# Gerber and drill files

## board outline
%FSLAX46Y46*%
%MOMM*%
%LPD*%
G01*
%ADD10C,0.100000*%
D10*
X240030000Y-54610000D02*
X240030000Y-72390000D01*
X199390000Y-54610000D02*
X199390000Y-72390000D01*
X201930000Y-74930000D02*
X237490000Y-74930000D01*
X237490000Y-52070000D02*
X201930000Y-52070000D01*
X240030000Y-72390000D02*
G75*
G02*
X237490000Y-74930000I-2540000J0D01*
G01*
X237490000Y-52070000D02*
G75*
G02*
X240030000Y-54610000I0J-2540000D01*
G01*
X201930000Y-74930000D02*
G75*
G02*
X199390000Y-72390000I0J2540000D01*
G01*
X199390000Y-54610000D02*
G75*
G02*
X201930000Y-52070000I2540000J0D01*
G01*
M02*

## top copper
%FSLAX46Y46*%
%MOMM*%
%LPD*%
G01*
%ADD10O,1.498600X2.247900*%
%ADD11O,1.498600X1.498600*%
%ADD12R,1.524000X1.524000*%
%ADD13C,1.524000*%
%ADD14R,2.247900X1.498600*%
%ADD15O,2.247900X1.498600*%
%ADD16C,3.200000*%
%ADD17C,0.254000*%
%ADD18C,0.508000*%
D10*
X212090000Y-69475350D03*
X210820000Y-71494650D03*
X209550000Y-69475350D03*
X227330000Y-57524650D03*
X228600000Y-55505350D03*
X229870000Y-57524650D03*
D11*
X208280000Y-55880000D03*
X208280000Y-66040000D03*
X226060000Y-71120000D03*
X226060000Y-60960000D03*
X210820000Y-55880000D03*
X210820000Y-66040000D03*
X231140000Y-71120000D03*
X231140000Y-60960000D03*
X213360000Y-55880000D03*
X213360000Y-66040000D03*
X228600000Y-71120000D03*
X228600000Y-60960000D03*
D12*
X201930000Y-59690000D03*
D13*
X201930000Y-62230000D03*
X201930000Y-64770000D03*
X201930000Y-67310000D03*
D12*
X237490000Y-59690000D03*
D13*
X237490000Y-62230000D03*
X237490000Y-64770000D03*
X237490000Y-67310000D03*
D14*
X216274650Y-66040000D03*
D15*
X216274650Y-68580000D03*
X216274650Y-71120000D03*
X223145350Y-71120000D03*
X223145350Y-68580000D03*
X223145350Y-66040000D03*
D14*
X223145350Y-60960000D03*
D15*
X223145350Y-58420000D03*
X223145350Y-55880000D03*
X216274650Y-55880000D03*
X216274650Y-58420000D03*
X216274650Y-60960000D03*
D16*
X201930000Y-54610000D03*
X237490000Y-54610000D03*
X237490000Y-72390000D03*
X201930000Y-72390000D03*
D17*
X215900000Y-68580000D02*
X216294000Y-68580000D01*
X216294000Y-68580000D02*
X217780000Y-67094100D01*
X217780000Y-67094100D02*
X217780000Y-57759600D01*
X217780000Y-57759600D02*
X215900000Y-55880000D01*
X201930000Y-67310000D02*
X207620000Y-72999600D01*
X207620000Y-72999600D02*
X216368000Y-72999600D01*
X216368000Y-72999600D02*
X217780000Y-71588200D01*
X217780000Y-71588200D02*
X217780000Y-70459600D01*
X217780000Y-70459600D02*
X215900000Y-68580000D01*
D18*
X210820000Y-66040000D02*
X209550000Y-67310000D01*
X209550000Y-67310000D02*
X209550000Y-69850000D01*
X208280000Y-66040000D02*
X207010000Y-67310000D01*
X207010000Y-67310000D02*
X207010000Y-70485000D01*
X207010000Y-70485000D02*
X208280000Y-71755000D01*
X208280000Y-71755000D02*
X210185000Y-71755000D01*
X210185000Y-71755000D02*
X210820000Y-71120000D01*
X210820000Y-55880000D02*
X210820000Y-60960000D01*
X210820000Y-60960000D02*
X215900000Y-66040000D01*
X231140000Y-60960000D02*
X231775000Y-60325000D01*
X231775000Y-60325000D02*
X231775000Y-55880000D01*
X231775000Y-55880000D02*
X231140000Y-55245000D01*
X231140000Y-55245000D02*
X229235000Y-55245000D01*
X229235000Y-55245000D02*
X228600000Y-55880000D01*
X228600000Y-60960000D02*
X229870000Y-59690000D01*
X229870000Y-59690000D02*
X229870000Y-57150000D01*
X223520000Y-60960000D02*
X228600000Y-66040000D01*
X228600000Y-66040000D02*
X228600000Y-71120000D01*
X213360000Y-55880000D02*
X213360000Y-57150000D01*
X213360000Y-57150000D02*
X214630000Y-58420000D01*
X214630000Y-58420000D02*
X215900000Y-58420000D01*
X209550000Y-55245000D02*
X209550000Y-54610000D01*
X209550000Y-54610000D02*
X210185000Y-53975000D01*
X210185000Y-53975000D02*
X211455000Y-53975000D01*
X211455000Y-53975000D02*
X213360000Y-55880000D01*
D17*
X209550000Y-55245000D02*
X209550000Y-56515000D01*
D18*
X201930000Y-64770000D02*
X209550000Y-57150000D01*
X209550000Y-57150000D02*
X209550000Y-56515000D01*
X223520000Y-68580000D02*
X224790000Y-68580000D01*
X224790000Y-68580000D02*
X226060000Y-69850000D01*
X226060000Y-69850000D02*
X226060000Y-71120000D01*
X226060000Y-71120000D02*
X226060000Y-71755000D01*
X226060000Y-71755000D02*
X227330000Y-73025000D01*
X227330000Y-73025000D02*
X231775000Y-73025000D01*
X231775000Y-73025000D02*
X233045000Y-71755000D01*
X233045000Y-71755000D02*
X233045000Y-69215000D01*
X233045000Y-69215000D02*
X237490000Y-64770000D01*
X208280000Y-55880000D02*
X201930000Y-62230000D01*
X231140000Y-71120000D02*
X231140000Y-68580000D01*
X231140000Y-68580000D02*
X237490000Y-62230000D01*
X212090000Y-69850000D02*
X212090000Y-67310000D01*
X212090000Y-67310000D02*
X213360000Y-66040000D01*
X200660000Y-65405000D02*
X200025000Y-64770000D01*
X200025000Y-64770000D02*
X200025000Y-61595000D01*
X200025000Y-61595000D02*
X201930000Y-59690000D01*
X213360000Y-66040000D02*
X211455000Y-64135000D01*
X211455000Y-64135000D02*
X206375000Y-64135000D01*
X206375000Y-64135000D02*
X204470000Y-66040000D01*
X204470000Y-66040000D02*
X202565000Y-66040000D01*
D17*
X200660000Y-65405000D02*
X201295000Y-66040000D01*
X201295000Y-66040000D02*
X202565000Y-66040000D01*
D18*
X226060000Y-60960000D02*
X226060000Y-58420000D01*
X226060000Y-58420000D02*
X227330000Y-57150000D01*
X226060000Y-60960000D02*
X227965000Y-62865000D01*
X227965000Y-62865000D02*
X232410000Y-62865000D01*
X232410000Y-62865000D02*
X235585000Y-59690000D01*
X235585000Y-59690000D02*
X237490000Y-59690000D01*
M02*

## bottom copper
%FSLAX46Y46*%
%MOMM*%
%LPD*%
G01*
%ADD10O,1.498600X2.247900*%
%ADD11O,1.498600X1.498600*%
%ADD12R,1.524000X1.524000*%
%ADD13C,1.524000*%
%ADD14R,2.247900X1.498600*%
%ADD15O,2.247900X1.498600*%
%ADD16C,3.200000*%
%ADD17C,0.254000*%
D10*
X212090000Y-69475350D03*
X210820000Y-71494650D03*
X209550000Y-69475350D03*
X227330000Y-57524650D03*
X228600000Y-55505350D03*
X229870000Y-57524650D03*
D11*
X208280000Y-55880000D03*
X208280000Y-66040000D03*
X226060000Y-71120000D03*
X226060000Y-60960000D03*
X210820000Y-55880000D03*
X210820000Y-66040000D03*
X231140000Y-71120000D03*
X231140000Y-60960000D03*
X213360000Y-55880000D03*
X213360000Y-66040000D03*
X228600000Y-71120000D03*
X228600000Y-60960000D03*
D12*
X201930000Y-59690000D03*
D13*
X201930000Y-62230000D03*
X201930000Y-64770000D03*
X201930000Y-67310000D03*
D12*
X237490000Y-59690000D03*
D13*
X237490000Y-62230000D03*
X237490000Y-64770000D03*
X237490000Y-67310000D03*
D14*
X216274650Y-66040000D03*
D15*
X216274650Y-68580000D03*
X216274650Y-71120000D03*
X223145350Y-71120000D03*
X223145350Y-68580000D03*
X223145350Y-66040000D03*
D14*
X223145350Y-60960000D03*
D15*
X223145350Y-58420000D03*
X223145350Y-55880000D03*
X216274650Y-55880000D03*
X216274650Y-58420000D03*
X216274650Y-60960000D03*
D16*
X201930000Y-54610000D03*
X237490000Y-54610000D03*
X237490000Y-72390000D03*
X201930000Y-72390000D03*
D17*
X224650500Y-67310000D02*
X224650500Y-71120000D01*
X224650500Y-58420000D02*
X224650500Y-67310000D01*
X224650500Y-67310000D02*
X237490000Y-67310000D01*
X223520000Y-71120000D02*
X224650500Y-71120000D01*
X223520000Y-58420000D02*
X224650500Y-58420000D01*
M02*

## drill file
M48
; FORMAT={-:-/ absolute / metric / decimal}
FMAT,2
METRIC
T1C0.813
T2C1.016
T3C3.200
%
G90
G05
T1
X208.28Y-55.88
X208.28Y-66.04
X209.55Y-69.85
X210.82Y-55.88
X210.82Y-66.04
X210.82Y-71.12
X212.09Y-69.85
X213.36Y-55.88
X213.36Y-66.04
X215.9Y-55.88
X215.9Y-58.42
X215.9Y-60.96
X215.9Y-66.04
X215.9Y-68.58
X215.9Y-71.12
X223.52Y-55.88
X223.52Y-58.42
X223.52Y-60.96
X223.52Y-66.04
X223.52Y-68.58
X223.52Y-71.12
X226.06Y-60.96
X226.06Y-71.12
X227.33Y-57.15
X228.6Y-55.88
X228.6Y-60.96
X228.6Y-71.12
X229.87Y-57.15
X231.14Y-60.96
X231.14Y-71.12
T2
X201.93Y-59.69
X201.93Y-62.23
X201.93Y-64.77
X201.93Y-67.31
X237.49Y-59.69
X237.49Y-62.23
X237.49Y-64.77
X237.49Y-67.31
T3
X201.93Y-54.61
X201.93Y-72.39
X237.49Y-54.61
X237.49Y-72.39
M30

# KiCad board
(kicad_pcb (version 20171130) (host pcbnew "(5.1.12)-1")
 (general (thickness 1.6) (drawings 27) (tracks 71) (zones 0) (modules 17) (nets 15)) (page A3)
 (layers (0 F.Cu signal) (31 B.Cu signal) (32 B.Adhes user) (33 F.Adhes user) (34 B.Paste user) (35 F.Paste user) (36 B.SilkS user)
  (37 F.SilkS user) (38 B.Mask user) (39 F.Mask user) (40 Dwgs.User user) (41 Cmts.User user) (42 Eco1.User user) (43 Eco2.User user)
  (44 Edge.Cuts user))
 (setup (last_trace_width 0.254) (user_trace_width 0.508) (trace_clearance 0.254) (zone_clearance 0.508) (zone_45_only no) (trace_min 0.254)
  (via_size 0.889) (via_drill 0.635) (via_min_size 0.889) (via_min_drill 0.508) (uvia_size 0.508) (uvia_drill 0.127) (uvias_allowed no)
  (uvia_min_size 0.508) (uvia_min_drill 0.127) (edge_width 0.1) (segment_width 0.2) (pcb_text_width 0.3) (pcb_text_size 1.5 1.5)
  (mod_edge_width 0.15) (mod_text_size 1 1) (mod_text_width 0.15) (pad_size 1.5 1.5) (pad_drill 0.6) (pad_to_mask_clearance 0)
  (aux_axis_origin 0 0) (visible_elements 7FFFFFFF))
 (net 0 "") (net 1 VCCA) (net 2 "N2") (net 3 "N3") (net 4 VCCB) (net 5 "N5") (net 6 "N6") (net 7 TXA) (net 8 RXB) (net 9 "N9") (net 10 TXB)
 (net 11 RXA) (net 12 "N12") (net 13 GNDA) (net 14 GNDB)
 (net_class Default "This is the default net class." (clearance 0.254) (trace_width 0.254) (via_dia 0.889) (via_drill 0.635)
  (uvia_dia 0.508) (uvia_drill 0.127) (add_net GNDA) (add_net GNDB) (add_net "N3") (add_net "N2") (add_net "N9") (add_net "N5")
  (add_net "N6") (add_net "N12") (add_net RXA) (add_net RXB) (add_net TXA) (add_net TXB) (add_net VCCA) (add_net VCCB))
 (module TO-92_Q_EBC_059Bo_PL (layer F.Cu) (at 212.09 69.85)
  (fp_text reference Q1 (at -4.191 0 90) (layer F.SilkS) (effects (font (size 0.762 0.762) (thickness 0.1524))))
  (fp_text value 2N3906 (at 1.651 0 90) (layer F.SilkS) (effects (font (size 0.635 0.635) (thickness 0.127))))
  (pad 1 thru_hole oval (at 0 0) (size 1.4986 2.2479) (drill 0.8128 (offset 0 -0.37465)) (layers *.Cu *.Mask F.SilkS) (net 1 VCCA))
  (pad 2 thru_hole oval (at -1.27 1.27) (size 1.4986 2.2479) (drill 0.8128 (offset 0 0.37465)) (layers *.Cu *.Mask F.SilkS) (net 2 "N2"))
  (pad 3 thru_hole oval (at -2.54 0) (size 1.4986 2.2479) (drill 0.8128 (offset 0 -0.37465)) (layers *.Cu *.Mask F.SilkS) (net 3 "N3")))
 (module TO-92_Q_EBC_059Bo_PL (layer F.Cu) (at 227.33 57.15 180)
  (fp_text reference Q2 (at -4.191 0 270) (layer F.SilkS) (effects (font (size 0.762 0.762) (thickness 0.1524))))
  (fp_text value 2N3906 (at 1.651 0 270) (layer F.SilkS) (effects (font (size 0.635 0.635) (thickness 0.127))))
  (pad 1 thru_hole oval (at 0 0 180) (size 1.4986 2.2479) (drill 0.8128 (offset 0 -0.37465)) (layers *.Cu *.Mask F.SilkS) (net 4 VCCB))
  (pad 2 thru_hole oval (at -1.27 1.27 180) (size 1.4986 2.2479) (drill 0.8128 (offset 0 0.37465)) (layers *.Cu *.Mask F.SilkS) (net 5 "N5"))
  (pad 3 thru_hole oval (at -2.54 0 180) (size 1.4986 2.2479) (drill 0.8128 (offset 0 -0.37465)) (layers *.Cu *.Mask F.SilkS) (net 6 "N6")))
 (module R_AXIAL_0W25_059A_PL (layer F.Cu) (at 208.28 55.88 270) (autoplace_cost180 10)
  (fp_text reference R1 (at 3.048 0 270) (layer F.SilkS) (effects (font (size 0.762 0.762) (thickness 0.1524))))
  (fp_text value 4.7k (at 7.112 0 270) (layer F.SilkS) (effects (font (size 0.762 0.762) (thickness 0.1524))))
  (pad 1 thru_hole oval (at 0 0 270) (size 1.4986 1.4986) (drill 0.8128) (layers *.Cu *.Mask F.SilkS) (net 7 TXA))
  (pad 2 thru_hole oval (at 10.16 0 270) (size 1.4986 1.4986) (drill 0.8128) (layers *.Cu *.Mask F.SilkS) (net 2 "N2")))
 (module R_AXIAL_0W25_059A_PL (layer F.Cu) (at 226.06 71.12 90) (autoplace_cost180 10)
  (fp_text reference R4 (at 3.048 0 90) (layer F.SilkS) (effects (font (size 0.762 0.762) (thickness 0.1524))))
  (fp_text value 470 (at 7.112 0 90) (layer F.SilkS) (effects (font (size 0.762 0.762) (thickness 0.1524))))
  (pad 1 thru_hole oval (at 0 0 90) (size 1.4986 1.4986) (drill 0.8128) (layers *.Cu *.Mask F.SilkS) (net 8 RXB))
  (pad 2 thru_hole oval (at 10.16 0 90) (size 1.4986 1.4986) (drill 0.8128) (layers *.Cu *.Mask F.SilkS) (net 4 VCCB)))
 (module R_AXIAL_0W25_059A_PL (layer F.Cu) (at 210.82 55.88 270) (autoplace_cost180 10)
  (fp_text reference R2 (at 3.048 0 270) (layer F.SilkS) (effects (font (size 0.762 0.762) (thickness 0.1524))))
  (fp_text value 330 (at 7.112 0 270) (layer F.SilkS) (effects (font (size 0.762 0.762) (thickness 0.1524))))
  (pad 1 thru_hole oval (at 0 0 270) (size 1.4986 1.4986) (drill 0.8128) (layers *.Cu *.Mask F.SilkS) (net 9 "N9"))
  (pad 2 thru_hole oval (at 10.16 0 270) (size 1.4986 1.4986) (drill 0.8128) (layers *.Cu *.Mask F.SilkS) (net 3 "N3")))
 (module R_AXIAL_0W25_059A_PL (layer F.Cu) (at 231.14 71.12 90) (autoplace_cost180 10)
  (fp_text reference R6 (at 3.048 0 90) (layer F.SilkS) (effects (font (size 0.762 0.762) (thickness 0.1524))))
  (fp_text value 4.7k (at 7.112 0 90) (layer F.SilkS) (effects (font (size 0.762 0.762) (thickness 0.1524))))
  (pad 1 thru_hole oval (at 0 0 90) (size 1.4986 1.4986) (drill 0.8128) (layers *.Cu *.Mask F.SilkS) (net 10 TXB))
  (pad 2 thru_hole oval (at 10.16 0 90) (size 1.4986 1.4986) (drill 0.8128) (layers *.Cu *.Mask F.SilkS) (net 5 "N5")))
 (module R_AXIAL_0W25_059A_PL (layer F.Cu) (at 213.36 55.88 270) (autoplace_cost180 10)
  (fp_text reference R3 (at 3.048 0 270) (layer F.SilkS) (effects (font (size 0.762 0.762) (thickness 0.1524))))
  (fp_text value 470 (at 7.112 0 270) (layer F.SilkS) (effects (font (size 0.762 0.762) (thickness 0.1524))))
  (pad 1 thru_hole oval (at 0 0 270) (size 1.4986 1.4986) (drill 0.8128) (layers *.Cu *.Mask F.SilkS) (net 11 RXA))
  (pad 2 thru_hole oval (at 10.16 0 270) (size 1.4986 1.4986) (drill 0.8128) (layers *.Cu *.Mask F.SilkS) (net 1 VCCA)))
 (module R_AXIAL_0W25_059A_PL (layer F.Cu) (at 228.6 71.12 90) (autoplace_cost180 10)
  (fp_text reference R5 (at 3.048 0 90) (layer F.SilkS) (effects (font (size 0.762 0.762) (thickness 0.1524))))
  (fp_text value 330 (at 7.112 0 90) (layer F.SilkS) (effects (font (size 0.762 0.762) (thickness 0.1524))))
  (pad 1 thru_hole oval (at 0 0 90) (size 1.4986 1.4986) (drill 0.8128) (layers *.Cu *.Mask F.SilkS) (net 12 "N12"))
  (pad 2 thru_hole oval (at 10.16 0 90) (size 1.4986 1.4986) (drill 0.8128) (layers *.Cu *.Mask F.SilkS) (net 6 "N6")))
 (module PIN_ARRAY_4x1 (layer F.Cu) (at 201.93 63.5 270)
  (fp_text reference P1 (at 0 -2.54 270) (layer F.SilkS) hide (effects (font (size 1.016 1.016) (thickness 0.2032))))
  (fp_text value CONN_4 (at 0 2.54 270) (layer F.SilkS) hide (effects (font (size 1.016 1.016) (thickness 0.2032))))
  (pad 1 thru_hole rect (at -3.81 0 270) (size 1.524 1.524) (drill 1.016) (layers *.Cu *.Mask F.SilkS) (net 1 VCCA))
  (pad 2 thru_hole circle (at -1.27 0 270) (size 1.524 1.524) (drill 1.016) (layers *.Cu *.Mask F.SilkS) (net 7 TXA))
  (pad 3 thru_hole circle (at 1.27 0 270) (size 1.524 1.524) (drill 1.016) (layers *.Cu *.Mask F.SilkS) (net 11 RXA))
  (pad 4 thru_hole circle (at 3.81 0 270) (size 1.524 1.524) (drill 1.016) (layers *.Cu *.Mask F.SilkS) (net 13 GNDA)))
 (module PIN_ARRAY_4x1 (layer F.Cu) (at 237.49 63.5 270)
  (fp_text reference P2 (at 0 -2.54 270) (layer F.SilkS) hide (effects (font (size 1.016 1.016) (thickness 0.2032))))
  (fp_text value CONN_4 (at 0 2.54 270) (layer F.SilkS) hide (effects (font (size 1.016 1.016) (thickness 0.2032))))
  (pad 1 thru_hole rect (at -3.81 0 270) (size 1.524 1.524) (drill 1.016) (layers *.Cu *.Mask F.SilkS) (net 4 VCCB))
  (pad 2 thru_hole circle (at -1.27 0 270) (size 1.524 1.524) (drill 1.016) (layers *.Cu *.Mask F.SilkS) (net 10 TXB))
  (pad 3 thru_hole circle (at 1.27 0 270) (size 1.524 1.524) (drill 1.016) (layers *.Cu *.Mask F.SilkS) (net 8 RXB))
  (pad 4 thru_hole circle (at 3.81 0 270) (size 1.524 1.524) (drill 1.016) (layers *.Cu *.Mask F.SilkS) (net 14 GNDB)))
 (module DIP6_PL (layer F.Cu) (at 215.9 66.04 270)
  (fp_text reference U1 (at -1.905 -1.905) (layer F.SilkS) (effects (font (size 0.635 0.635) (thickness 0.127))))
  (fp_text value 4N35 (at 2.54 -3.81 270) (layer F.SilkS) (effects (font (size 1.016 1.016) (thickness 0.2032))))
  (pad 1 thru_hole rect (at 0 0 270) (size 1.4986 2.2479) (drill 0.8128 (offset 0 -0.37465)) (layers *.Cu *.Mask F.SilkS) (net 9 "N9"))
  (pad 2 thru_hole oval (at 2.54 0 270) (size 1.4986 2.2479) (drill 0.8128 (offset 0 -0.37465)) (layers *.Cu *.Mask F.SilkS) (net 13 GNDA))
  (pad 3 thru_hole oval (at 5.08 0 270) (size 1.4986 2.2479) (drill 0.8128 (offset 0 -0.37465)) (layers *.Cu *.Mask F.SilkS))
  (pad 4 thru_hole oval (at 5.08 -7.62 270) (size 1.4986 2.2479) (drill 0.8128 (offset 0 0.37465)) (layers *.Cu *.Mask F.SilkS)
   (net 14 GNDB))
  (pad 5 thru_hole oval (at 2.54 -7.62 270) (size 1.4986 2.2479) (drill 0.8128 (offset 0 0.37465)) (layers *.Cu *.Mask F.SilkS) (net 8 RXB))
  (pad 6 thru_hole oval (at 0 -7.62 270) (size 1.4986 2.2479) (drill 0.8128 (offset 0 0.37465)) (layers *.Cu *.Mask F.SilkS)))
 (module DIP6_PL (layer F.Cu) (at 223.52 60.96 90)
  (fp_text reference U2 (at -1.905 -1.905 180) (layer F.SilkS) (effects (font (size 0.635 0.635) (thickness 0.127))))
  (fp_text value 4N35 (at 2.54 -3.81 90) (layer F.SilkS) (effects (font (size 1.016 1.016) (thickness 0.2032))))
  (pad 1 thru_hole rect (at 0 0 90) (size 1.4986 2.2479) (drill 0.8128 (offset 0 -0.37465)) (layers *.Cu *.Mask F.SilkS) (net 12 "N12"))
  (pad 2 thru_hole oval (at 2.54 0 90) (size 1.4986 2.2479) (drill 0.8128 (offset 0 -0.37465)) (layers *.Cu *.Mask F.SilkS) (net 14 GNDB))
  (pad 3 thru_hole oval (at 5.08 0 90) (size 1.4986 2.2479) (drill 0.8128 (offset 0 -0.37465)) (layers *.Cu *.Mask F.SilkS))
  (pad 4 thru_hole oval (at 5.08 -7.62 90) (size 1.4986 2.2479) (drill 0.8128 (offset 0 0.37465)) (layers *.Cu *.Mask F.SilkS) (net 13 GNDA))
  (pad 5 thru_hole oval (at 2.54 -7.62 90) (size 1.4986 2.2479) (drill 0.8128 (offset 0 0.37465)) (layers *.Cu *.Mask F.SilkS) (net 11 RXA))
  (pad 6 thru_hole oval (at 0 -7.62 90) (size 1.4986 2.2479) (drill 0.8128 (offset 0 0.37465)) (layers *.Cu *.Mask F.SilkS)))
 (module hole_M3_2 (layer F.Cu) (at 201.93 54.61)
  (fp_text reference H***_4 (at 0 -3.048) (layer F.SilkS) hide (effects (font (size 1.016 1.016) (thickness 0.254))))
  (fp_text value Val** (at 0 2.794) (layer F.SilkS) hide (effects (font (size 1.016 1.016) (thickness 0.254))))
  (pad 1 thru_hole circle (at 0 0) (size 3.2 3.2) (drill 3.2) (layers *.Cu *.Mask F.SilkS)))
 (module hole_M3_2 (layer F.Cu) (at 237.49 54.61)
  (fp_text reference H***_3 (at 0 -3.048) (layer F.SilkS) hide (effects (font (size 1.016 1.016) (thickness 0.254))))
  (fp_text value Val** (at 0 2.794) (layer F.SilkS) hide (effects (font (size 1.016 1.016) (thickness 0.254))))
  (pad 1 thru_hole circle (at 0 0) (size 3.2 3.2) (drill 3.2) (layers *.Cu *.Mask F.SilkS)))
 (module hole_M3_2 (layer F.Cu) (at 237.49 72.39)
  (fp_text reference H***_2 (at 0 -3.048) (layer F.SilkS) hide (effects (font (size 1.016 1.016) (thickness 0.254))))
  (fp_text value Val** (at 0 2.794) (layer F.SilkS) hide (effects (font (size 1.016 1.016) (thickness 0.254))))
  (pad 1 thru_hole circle (at 0 0) (size 3.2 3.2) (drill 3.2) (layers *.Cu *.Mask F.SilkS)))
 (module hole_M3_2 (layer F.Cu) (at 201.93 72.39)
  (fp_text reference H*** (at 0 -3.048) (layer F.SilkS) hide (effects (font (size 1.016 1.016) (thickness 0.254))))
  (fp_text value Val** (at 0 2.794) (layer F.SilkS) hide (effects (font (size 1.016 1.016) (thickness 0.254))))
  (pad 1 thru_hole circle (at 0 0) (size 3.2 3.2) (drill 3.2) (layers *.Cu *.Mask F.SilkS)))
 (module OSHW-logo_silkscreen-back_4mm (layer F.Cu) (at 210.82 60.325)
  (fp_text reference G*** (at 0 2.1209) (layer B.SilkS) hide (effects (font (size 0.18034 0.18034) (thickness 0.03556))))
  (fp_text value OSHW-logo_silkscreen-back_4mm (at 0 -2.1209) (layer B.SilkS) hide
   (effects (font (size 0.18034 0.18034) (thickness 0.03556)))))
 (gr_line (start 240.03 54.61) (end 240.03 72.39) (angle 90) (layer Edge.Cuts) (width 0.1))
 (gr_line (start 199.39 54.61) (end 199.39 72.39) (angle 90) (layer Edge.Cuts) (width 0.1))
 (gr_line (start 201.93 74.93) (end 237.49 74.93) (angle 90) (layer Edge.Cuts) (width 0.1))
 (gr_line (start 237.49 52.07) (end 201.93 52.07) (angle 90) (layer Edge.Cuts) (width 0.1))
 (gr_arc (start 237.49 72.39) (end 240.03 72.39) (angle 90) (layer Edge.Cuts) (width 0.1))
 (gr_arc (start 237.49 54.61) (end 237.49 52.07) (angle 90) (layer Edge.Cuts) (width 0.1))
 (gr_arc (start 201.93 72.39) (end 201.93 74.93) (angle 90) (layer Edge.Cuts) (width 0.1))
 (gr_arc (start 201.93 54.61) (end 199.39 54.61) (angle 90) (layer Edge.Cuts) (width 0.1))
 (segment (start 215.9 68.58) (end 216.294 68.58) (width 0.254) (layer F.Cu) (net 13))
 (segment (start 216.294 68.58) (end 217.78 67.0941) (width 0.254) (layer F.Cu) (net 13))
 (segment (start 217.78 67.0941) (end 217.78 57.7596) (width 0.254) (layer F.Cu) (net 13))
 (segment (start 217.78 57.7596) (end 215.9 55.88) (width 0.254) (layer F.Cu) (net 13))
 (segment (start 201.93 67.31) (end 207.62 72.9996) (width 0.254) (layer F.Cu) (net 13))
 (segment (start 207.62 72.9996) (end 216.368 72.9996) (width 0.254) (layer F.Cu) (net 13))
 (segment (start 216.368 72.9996) (end 217.78 71.5882) (width 0.254) (layer F.Cu) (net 13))
 (segment (start 217.78 71.5882) (end 217.78 70.4596) (width 0.254) (layer F.Cu) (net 13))
 (segment (start 217.78 70.4596) (end 215.9 68.58) (width 0.254) (layer F.Cu) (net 13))
 (segment (start 224.6505 67.31) (end 224.6505 71.12) (width 0.254) (layer B.Cu) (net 14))
 (segment (start 224.6505 58.42) (end 224.6505 67.31) (width 0.254) (layer B.Cu) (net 14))
 (segment (start 224.6505 67.31) (end 237.49 67.31) (width 0.254) (layer B.Cu) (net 14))
 (segment (start 223.52 71.12) (end 224.6505 71.12) (width 0.254) (layer B.Cu) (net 14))
 (segment (start 223.52 58.42) (end 224.6505 58.42) (width 0.254) (layer B.Cu) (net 14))
 (segment (start 210.82 66.04) (end 209.55 67.31) (width 0.508) (layer F.Cu) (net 3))
 (segment (start 209.55 67.31) (end 209.55 69.85) (width 0.508) (layer F.Cu) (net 3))
 (segment (start 208.28 66.04) (end 207.01 67.31) (width 0.508) (layer F.Cu) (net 2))
 (segment (start 207.01 67.31) (end 207.01 70.485) (width 0.508) (layer F.Cu) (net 2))
 (segment (start 207.01 70.485) (end 208.28 71.755) (width 0.508) (layer F.Cu) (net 2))
 (segment (start 208.28 71.755) (end 210.185 71.755) (width 0.508) (layer F.Cu) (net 2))
 (segment (start 210.185 71.755) (end 210.82 71.12) (width 0.508) (layer F.Cu) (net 2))
 (segment (start 210.82 55.88) (end 210.82 60.96) (width 0.508) (layer F.Cu) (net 9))
 (segment (start 210.82 60.96) (end 215.9 66.04) (width 0.508) (layer F.Cu) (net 9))
 (segment (start 231.14 60.96) (end 231.775 60.325) (width 0.508) (layer F.Cu) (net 5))
 (segment (start 231.775 60.325) (end 231.775 55.88) (width 0.508) (layer F.Cu) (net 5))
 (segment (start 231.775 55.88) (end 231.14 55.245) (width 0.508) (layer F.Cu) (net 5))
 (segment (start 231.14 55.245) (end 229.235 55.245) (width 0.508) (layer F.Cu) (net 5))
 (segment (start 229.235 55.245) (end 228.6 55.88) (width 0.508) (layer F.Cu) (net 5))
 (segment (start 228.6 60.96) (end 229.87 59.69) (width 0.508) (layer F.Cu) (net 6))
 (segment (start 229.87 59.69) (end 229.87 57.15) (width 0.508) (layer F.Cu) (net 6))
 (segment (start 223.52 60.96) (end 228.6 66.04) (width 0.508) (layer F.Cu) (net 12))
 (segment (start 228.6 66.04) (end 228.6 71.12) (width 0.508) (layer F.Cu) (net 12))
 (segment (start 213.36 55.88) (end 213.36 57.15) (width 0.508) (layer F.Cu) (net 11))
 (segment (start 213.36 57.15) (end 214.63 58.42) (width 0.508) (layer F.Cu) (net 11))
 (segment (start 214.63 58.42) (end 215.9 58.42) (width 0.508) (layer F.Cu) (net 11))
 (segment (start 209.55 55.245) (end 209.55 54.61) (width 0.508) (layer F.Cu) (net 11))
 (segment (start 209.55 54.61) (end 210.185 53.975) (width 0.508) (layer F.Cu) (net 11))
 (segment (start 210.185 53.975) (end 211.455 53.975) (width 0.508) (layer F.Cu) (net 11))
 (segment (start 211.455 53.975) (end 213.36 55.88) (width 0.508) (layer F.Cu) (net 11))
 (segment (start 209.55 55.245) (end 209.55 56.515) (width 0.254) (layer F.Cu) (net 11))
 (segment (start 201.93 64.77) (end 209.55 57.15) (width 0.508) (layer F.Cu) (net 11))
 (segment (start 209.55 57.15) (end 209.55 56.515) (width 0.508) (layer F.Cu) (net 11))
 (segment (start 223.52 68.58) (end 224.79 68.58) (width 0.508) (layer F.Cu) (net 8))
 (segment (start 224.79 68.58) (end 226.06 69.85) (width 0.508) (layer F.Cu) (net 8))
 (segment (start 226.06 69.85) (end 226.06 71.12) (width 0.508) (layer F.Cu) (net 8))
 (segment (start 226.06 71.12) (end 226.06 71.755) (width 0.508) (layer F.Cu) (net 8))
 (segment (start 226.06 71.755) (end 227.33 73.025) (width 0.508) (layer F.Cu) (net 8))
 (segment (start 227.33 73.025) (end 231.775 73.025) (width 0.508) (layer F.Cu) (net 8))
 (segment (start 231.775 73.025) (end 233.045 71.755) (width 0.508) (layer F.Cu) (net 8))
 (segment (start 233.045 71.755) (end 233.045 69.215) (width 0.508) (layer F.Cu) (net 8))
 (segment (start 233.045 69.215) (end 237.49 64.77) (width 0.508) (layer F.Cu) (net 8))
 (segment (start 208.28 55.88) (end 201.93 62.23) (width 0.508) (layer F.Cu) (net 7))
 (segment (start 231.14 71.12) (end 231.14 68.58) (width 0.508) (layer F.Cu) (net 10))
 (segment (start 231.14 68.58) (end 237.49 62.23) (width 0.508) (layer F.Cu) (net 10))
 (segment (start 212.09 69.85) (end 212.09 67.31) (width 0.508) (layer F.Cu) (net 1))
 (segment (start 212.09 67.31) (end 213.36 66.04) (width 0.508) (layer F.Cu) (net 1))
 (segment (start 200.66 65.405) (end 200.025 64.77) (width 0.508) (layer F.Cu) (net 1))
 (segment (start 200.025 64.77) (end 200.025 61.595) (width 0.508) (layer F.Cu) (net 1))
 (segment (start 200.025 61.595) (end 201.93 59.69) (width 0.508) (layer F.Cu) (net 1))
 (segment (start 213.36 66.04) (end 211.455 64.135) (width 0.508) (layer F.Cu) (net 1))
 (segment (start 211.455 64.135) (end 206.375 64.135) (width 0.508) (layer F.Cu) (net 1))
 (segment (start 206.375 64.135) (end 204.47 66.04) (width 0.508) (layer F.Cu) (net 1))
 (segment (start 204.47 66.04) (end 202.565 66.04) (width 0.508) (layer F.Cu) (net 1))
 (segment (start 200.66 65.405) (end 201.295 66.04) (width 0.254) (layer F.Cu) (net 1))
 (segment (start 201.295 66.04) (end 202.565 66.04) (width 0.254) (layer F.Cu) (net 1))
 (segment (start 226.06 60.96) (end 226.06 58.42) (width 0.508) (layer F.Cu) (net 4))
 (segment (start 226.06 58.42) (end 227.33 57.15) (width 0.508) (layer F.Cu) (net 4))
 (segment (start 226.06 60.96) (end 227.965 62.865) (width 0.508) (layer F.Cu) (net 4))
 (segment (start 227.965 62.865) (end 232.41 62.865) (width 0.508) (layer F.Cu) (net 4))
 (segment (start 232.41 62.865) (end 235.585 59.69) (width 0.508) (layer F.Cu) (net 4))
 (segment (start 235.585 59.69) (end 237.49 59.69) (width 0.508) (layer F.Cu) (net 4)))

